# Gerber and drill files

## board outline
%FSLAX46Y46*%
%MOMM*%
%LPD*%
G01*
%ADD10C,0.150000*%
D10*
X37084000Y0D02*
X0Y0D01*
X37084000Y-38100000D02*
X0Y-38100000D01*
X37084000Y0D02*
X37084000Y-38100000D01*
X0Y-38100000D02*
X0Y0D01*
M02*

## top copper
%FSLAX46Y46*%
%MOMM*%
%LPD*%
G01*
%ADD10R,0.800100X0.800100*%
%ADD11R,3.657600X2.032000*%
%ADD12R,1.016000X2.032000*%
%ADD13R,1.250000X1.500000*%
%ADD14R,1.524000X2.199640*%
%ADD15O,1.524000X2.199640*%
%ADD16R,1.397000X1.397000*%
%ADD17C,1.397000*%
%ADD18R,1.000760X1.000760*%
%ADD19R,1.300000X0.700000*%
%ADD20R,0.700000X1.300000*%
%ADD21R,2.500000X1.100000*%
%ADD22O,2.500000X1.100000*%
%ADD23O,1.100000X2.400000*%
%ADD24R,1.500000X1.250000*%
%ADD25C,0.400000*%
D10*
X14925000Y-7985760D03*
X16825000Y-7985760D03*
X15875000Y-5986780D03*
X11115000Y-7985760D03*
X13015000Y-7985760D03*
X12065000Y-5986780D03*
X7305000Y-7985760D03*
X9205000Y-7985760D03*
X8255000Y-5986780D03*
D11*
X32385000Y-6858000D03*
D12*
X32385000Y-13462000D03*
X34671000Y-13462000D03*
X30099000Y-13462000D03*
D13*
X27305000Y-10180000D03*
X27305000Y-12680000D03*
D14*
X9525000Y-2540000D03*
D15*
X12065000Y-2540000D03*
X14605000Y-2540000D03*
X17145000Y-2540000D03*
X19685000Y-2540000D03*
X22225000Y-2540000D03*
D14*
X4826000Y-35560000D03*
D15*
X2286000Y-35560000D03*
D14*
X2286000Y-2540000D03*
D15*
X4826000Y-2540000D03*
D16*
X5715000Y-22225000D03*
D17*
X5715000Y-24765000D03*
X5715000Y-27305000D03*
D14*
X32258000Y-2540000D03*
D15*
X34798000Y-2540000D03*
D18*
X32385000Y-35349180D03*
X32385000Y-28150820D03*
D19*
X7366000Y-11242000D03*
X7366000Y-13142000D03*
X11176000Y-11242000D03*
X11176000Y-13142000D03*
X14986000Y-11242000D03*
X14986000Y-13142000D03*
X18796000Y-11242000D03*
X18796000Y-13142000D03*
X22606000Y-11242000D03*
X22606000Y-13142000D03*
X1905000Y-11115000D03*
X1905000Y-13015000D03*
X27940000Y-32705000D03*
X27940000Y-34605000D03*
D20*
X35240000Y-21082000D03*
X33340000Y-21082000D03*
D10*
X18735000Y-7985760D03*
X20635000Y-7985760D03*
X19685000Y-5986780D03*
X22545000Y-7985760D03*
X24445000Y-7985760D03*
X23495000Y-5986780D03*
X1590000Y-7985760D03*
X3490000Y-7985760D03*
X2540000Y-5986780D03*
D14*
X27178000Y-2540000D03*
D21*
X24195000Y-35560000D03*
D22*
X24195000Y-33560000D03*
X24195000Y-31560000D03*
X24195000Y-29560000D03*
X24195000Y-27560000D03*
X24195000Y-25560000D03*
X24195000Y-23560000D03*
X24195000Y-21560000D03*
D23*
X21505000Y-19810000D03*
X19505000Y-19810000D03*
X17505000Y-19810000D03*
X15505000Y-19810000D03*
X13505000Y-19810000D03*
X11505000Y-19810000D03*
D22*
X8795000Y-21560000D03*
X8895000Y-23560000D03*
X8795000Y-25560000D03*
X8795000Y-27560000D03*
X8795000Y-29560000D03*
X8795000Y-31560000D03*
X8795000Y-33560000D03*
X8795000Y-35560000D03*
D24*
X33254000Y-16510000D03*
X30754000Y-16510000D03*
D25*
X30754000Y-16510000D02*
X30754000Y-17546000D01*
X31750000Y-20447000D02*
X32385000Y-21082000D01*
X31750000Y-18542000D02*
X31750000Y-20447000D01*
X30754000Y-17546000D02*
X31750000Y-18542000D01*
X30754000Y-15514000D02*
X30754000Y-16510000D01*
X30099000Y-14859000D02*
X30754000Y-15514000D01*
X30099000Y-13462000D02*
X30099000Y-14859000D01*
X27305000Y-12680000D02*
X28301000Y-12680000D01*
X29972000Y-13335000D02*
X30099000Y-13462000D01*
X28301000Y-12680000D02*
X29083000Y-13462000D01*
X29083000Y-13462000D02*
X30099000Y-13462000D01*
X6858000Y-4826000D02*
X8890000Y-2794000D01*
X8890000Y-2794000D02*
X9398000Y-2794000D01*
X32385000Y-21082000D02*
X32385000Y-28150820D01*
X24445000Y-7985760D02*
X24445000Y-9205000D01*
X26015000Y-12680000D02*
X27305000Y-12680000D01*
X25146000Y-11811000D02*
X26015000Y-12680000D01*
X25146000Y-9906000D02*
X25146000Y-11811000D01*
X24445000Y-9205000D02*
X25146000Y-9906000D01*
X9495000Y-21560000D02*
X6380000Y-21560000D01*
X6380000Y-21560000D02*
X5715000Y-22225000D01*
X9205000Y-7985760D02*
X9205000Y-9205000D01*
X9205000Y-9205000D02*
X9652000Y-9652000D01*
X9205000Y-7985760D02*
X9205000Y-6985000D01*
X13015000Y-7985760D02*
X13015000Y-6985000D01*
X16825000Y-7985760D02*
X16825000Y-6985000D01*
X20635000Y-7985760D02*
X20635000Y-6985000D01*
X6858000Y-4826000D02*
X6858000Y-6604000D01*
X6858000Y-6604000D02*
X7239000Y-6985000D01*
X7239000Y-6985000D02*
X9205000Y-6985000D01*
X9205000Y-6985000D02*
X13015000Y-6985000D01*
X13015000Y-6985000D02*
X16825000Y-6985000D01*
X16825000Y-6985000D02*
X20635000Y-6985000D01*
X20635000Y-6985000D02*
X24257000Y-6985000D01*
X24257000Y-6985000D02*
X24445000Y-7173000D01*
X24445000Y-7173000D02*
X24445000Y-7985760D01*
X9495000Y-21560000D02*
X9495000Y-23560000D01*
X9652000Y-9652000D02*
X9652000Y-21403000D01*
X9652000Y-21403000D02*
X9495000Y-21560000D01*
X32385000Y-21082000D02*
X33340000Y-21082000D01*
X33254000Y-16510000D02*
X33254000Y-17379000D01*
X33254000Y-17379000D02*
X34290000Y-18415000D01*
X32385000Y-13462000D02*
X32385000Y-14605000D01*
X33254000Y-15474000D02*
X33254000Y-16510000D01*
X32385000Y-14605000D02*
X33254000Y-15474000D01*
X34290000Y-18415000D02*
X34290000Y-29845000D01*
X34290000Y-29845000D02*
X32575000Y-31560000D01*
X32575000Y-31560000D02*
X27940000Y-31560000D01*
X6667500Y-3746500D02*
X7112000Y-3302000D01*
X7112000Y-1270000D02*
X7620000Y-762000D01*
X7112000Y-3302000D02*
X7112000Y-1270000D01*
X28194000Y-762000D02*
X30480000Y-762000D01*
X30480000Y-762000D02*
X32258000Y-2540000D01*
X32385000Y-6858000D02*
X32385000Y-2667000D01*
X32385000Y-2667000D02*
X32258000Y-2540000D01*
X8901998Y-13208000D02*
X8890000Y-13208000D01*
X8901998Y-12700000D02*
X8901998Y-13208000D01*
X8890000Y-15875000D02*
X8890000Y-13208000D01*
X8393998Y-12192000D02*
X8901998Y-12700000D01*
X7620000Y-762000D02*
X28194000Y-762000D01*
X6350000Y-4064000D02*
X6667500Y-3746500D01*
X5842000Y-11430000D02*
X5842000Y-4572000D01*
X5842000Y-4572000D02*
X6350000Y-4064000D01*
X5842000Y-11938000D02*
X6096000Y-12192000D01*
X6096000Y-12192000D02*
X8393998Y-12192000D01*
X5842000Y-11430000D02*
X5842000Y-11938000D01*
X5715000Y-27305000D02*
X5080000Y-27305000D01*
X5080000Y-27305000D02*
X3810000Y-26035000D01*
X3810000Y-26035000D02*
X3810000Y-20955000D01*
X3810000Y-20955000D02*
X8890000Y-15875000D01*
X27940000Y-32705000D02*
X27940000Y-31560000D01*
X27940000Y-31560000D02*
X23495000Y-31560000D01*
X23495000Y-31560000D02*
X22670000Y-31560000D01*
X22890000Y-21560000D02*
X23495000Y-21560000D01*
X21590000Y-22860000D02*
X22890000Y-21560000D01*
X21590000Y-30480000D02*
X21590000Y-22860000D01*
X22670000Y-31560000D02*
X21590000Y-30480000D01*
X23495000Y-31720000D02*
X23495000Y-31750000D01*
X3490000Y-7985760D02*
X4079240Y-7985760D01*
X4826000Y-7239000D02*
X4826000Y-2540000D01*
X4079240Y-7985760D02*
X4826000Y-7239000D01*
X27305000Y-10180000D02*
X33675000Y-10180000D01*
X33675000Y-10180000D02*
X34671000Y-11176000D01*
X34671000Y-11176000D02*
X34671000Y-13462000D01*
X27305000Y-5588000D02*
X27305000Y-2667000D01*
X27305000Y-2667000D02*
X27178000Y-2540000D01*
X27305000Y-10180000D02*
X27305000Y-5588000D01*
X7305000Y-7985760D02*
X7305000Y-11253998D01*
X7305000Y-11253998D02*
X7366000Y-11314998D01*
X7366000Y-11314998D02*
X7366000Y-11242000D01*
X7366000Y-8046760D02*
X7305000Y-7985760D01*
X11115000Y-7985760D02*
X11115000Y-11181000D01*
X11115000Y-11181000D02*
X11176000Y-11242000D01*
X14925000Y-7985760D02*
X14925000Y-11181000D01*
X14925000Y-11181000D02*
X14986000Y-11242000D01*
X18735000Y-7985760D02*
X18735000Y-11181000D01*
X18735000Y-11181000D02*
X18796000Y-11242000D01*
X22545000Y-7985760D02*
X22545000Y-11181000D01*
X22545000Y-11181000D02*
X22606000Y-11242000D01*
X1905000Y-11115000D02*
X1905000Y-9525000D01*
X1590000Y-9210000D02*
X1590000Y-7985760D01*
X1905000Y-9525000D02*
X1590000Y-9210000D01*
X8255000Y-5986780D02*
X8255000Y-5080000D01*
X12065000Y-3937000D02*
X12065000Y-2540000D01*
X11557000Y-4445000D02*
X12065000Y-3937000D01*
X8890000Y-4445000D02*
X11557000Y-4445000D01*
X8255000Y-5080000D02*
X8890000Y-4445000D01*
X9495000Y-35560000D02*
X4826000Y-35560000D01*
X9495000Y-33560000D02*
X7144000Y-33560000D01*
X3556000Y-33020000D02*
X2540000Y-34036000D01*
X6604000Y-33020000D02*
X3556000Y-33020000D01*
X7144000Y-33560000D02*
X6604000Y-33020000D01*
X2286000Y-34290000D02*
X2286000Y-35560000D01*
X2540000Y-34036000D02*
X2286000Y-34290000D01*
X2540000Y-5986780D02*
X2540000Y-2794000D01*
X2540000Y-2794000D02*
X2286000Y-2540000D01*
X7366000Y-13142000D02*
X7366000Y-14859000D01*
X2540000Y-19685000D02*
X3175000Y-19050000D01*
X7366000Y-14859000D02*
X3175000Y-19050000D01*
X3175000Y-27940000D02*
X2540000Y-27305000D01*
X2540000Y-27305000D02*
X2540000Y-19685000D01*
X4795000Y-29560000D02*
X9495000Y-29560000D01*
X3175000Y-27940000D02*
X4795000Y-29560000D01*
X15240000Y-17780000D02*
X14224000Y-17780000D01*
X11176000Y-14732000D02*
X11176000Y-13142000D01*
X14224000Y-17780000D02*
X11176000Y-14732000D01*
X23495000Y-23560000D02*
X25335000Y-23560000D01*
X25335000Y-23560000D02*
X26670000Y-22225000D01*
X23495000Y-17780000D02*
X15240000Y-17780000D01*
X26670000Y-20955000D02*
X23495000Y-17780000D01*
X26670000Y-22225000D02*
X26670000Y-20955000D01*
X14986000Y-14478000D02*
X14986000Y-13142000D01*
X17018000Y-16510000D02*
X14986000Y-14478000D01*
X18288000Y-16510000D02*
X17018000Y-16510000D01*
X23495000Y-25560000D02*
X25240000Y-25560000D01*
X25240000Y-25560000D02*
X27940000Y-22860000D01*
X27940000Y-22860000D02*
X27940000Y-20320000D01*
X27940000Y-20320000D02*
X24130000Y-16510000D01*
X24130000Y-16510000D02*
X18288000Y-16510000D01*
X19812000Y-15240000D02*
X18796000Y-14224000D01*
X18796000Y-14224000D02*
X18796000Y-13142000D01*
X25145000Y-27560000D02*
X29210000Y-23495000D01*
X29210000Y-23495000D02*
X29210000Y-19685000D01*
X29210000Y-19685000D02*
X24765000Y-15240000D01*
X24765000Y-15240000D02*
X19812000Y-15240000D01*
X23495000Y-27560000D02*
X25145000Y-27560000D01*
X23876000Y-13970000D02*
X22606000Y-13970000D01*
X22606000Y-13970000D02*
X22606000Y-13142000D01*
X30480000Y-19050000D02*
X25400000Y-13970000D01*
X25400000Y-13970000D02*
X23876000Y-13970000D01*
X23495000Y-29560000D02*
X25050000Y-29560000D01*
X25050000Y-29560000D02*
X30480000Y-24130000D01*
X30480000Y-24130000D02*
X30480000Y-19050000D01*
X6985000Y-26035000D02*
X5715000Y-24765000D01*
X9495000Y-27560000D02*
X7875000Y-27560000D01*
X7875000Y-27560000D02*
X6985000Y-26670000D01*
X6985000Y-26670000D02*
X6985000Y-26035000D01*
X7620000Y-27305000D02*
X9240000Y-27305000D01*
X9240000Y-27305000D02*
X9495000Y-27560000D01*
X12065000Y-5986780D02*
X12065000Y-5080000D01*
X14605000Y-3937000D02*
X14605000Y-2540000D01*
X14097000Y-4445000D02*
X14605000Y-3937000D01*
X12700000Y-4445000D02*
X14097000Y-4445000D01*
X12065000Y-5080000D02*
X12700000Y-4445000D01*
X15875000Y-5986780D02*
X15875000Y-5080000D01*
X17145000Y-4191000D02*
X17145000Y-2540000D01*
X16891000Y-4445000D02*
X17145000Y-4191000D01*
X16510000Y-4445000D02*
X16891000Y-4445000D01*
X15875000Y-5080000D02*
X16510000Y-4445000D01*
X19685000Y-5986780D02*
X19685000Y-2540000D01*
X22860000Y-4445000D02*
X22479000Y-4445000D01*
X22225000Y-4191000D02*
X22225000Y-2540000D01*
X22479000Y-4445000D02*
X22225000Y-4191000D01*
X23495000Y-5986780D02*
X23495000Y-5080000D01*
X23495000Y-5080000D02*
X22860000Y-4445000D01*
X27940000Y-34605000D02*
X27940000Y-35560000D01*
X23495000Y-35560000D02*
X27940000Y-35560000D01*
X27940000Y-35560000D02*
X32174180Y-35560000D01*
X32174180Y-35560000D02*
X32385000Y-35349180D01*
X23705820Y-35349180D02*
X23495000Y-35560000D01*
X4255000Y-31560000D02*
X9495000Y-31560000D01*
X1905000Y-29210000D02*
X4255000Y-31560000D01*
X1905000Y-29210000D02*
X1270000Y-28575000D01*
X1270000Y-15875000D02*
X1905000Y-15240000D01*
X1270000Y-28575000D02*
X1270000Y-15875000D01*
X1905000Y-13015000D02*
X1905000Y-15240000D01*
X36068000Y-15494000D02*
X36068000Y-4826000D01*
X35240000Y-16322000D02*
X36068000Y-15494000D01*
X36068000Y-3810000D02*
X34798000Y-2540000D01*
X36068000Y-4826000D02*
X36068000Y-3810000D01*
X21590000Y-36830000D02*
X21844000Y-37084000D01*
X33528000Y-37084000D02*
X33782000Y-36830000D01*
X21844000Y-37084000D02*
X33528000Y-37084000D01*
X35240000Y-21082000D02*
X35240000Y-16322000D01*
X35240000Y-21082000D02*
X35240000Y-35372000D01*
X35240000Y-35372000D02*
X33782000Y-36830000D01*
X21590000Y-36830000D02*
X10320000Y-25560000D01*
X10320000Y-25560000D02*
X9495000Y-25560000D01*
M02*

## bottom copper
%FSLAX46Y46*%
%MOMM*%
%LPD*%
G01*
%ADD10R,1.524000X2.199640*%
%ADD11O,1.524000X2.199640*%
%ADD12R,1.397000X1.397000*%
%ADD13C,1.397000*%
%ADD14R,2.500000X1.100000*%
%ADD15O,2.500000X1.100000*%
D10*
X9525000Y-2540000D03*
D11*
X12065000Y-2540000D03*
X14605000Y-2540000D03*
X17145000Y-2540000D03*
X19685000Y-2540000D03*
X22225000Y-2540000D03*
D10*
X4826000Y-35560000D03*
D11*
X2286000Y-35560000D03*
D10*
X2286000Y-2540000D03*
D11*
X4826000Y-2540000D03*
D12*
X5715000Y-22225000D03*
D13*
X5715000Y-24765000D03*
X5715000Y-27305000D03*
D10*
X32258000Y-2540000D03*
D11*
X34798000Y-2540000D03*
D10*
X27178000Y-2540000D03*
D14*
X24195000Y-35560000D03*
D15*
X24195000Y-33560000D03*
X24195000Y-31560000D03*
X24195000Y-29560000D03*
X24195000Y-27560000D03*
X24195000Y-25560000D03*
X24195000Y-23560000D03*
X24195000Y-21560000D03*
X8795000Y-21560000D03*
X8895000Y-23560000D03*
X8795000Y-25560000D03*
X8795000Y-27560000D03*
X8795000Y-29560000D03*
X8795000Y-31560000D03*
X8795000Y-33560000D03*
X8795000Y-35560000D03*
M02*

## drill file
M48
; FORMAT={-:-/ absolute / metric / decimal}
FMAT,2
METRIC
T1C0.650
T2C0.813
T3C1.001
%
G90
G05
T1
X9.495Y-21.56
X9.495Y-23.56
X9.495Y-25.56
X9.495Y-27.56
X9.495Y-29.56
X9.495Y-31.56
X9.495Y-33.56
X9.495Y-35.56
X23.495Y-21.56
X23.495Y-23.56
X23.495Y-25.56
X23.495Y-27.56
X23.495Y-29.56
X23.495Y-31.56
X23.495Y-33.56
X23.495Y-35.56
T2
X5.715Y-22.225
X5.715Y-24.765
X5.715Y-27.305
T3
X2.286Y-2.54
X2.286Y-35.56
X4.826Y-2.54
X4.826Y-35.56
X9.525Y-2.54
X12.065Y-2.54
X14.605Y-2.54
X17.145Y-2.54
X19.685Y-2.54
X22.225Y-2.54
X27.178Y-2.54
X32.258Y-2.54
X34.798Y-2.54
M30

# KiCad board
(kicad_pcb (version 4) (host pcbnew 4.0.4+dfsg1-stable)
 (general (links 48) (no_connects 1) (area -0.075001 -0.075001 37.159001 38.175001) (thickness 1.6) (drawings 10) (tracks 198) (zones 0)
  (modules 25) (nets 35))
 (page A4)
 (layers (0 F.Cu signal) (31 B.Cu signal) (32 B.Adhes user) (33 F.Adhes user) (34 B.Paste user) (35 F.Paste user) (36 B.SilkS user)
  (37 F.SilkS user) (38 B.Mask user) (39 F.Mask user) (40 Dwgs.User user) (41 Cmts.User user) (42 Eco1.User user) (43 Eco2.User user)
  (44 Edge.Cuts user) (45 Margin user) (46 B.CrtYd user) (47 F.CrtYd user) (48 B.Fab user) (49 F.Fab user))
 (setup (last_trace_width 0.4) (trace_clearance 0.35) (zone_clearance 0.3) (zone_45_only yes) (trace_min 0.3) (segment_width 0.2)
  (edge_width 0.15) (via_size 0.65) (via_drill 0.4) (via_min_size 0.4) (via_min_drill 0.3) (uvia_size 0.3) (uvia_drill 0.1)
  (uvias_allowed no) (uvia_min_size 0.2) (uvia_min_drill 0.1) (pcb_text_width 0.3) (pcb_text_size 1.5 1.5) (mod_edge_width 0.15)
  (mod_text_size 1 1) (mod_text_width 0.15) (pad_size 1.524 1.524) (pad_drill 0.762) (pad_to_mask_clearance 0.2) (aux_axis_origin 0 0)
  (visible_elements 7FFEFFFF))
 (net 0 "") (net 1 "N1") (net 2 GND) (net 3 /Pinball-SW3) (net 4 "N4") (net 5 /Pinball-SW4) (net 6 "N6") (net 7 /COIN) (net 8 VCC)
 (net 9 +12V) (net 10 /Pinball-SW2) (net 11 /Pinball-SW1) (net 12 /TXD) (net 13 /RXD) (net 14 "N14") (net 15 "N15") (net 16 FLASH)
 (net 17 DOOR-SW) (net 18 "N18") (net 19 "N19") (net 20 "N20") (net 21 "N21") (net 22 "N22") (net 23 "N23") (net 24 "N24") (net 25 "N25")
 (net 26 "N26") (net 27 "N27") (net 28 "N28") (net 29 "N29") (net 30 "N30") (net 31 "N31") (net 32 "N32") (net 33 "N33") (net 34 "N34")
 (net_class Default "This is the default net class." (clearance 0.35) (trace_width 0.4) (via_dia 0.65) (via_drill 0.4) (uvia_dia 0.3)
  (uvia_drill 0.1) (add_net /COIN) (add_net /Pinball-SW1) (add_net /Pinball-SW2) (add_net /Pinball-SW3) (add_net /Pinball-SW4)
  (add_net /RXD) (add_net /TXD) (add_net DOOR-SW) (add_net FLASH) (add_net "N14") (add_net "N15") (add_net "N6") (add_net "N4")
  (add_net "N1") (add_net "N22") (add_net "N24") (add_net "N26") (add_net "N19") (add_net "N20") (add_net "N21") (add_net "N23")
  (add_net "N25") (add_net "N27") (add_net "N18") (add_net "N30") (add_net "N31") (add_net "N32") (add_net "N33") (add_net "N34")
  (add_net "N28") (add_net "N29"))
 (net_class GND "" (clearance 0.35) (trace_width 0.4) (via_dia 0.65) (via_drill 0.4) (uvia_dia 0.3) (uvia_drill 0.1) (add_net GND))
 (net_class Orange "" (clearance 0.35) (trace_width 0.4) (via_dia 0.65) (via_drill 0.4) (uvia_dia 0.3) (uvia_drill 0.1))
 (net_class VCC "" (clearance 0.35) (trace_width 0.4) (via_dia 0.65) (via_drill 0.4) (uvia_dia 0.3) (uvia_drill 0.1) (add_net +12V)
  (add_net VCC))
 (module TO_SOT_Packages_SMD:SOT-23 (layer F.Cu) (at 15.875 6.985)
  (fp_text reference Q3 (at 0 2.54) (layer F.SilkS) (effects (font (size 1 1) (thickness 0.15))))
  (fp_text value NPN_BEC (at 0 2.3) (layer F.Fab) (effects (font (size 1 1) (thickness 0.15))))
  (pad 1 smd rect (at -0.95 1.00076) (size 0.8001 0.8001) (layers F.Cu F.Paste F.Mask) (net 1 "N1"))
  (pad 2 smd rect (at 0.95 1.00076) (size 0.8001 0.8001) (layers F.Cu F.Paste F.Mask) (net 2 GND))
  (pad 3 smd rect (at 0 -0.99822) (size 0.8001 0.8001) (layers F.Cu F.Paste F.Mask) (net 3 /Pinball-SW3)))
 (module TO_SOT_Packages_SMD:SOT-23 (layer F.Cu) (at 12.065 6.985)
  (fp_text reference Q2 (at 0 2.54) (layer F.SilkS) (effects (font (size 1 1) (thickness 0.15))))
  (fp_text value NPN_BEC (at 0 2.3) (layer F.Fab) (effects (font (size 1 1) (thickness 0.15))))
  (pad 1 smd rect (at -0.95 1.00076) (size 0.8001 0.8001) (layers F.Cu F.Paste F.Mask) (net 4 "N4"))
  (pad 2 smd rect (at 0.95 1.00076) (size 0.8001 0.8001) (layers F.Cu F.Paste F.Mask) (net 2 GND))
  (pad 3 smd rect (at 0 -0.99822) (size 0.8001 0.8001) (layers F.Cu F.Paste F.Mask) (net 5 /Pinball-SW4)))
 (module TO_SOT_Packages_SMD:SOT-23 (layer F.Cu) (at 8.255 6.985)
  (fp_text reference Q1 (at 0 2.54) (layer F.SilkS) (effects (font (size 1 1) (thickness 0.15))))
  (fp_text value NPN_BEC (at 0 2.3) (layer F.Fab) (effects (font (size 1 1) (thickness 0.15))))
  (pad 1 smd rect (at -0.95 1.00076) (size 0.8001 0.8001) (layers F.Cu F.Paste F.Mask) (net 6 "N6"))
  (pad 2 smd rect (at 0.95 1.00076) (size 0.8001 0.8001) (layers F.Cu F.Paste F.Mask) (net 2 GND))
  (pad 3 smd rect (at 0 -0.99822) (size 0.8001 0.8001) (layers F.Cu F.Paste F.Mask) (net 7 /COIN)))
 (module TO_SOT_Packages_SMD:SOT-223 (layer F.Cu) (at 32.385 10.16)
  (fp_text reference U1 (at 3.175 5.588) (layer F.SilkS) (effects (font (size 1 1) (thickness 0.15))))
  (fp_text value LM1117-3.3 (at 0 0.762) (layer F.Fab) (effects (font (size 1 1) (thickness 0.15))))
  (pad 4 smd rect (at 0 -3.302) (size 3.6576 2.032) (layers F.Cu F.Paste F.Mask) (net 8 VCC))
  (pad 2 smd rect (at 0 3.302) (size 1.016 2.032) (layers F.Cu F.Paste F.Mask) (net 8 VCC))
  (pad 3 smd rect (at 2.286 3.302) (size 1.016 2.032) (layers F.Cu F.Paste F.Mask) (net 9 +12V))
  (pad 1 smd rect (at -2.286 3.302) (size 1.016 2.032) (layers F.Cu F.Paste F.Mask) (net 2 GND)))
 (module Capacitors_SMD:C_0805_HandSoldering (layer F.Cu) (at 27.305 11.43 270)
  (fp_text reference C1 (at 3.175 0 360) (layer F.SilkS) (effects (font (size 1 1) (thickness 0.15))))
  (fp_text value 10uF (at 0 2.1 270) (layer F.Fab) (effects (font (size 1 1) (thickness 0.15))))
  (pad 1 smd rect (at -1.25 0 270) (size 1.5 1.25) (layers F.Cu F.Paste F.Mask) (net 9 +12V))
  (pad 2 smd rect (at 1.25 0 270) (size 1.5 1.25) (layers F.Cu F.Paste F.Mask) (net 2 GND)))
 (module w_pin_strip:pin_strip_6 (layer F.Cu) (at 15.875 2.54)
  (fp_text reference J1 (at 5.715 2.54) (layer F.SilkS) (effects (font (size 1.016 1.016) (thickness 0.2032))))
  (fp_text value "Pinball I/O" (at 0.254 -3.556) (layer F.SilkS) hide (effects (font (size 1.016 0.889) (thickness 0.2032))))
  (pad 1 thru_hole rect (at -6.35 0) (size 1.524 2.19964) (drill 1.00076) (layers *.Cu *.Mask F.SilkS) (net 2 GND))
  (pad 2 thru_hole oval (at -3.81 0) (size 1.524 2.19964) (drill 1.00076) (layers *.Cu *.Mask F.SilkS) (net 7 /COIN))
  (pad 3 thru_hole oval (at -1.27 0) (size 1.524 2.19964) (drill 1.00076) (layers *.Cu *.Mask F.SilkS) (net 5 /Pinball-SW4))
  (pad 4 thru_hole oval (at 1.27 0) (size 1.524 2.19964) (drill 1.00076) (layers *.Cu *.Mask F.SilkS) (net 3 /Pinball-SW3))
  (pad 5 thru_hole oval (at 3.81 0) (size 1.524 2.19964) (drill 1.00076) (layers *.Cu *.Mask F.SilkS) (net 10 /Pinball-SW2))
  (pad 6 thru_hole oval (at 6.35 0) (size 1.524 2.19964) (drill 1.00076) (layers *.Cu *.Mask F.SilkS) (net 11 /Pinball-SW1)))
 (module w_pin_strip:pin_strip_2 (layer F.Cu) (at 3.556 35.56 180)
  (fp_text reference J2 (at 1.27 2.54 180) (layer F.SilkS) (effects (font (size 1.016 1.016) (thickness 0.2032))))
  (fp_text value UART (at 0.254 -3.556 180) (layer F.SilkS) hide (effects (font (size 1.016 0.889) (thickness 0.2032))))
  (pad 1 thru_hole rect (at -1.27 0 180) (size 1.524 2.19964) (drill 1.00076) (layers *.Cu *.Mask F.SilkS) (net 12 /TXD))
  (pad 2 thru_hole oval (at 1.27 0 180) (size 1.524 2.19964) (drill 1.00076) (layers *.Cu *.Mask F.SilkS) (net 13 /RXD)))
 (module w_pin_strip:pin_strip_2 (layer F.Cu) (at 3.556 2.54)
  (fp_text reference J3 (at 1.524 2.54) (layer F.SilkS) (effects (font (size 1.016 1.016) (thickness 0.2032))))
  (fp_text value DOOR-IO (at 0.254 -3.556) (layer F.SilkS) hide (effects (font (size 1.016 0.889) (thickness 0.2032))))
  (pad 1 thru_hole rect (at -1.27 0) (size 1.524 2.19964) (drill 1.00076) (layers *.Cu *.Mask F.SilkS) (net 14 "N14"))
  (pad 2 thru_hole oval (at 1.27 0) (size 1.524 2.19964) (drill 1.00076) (layers *.Cu *.Mask F.SilkS) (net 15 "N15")))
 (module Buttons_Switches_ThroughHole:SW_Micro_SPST (layer F.Cu) (at 5.715 24.765 270)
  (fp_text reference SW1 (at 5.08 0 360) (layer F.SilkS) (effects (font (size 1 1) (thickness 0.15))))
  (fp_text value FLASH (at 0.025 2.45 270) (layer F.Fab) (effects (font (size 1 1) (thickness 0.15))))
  (pad 1 thru_hole rect (at -2.54 0 270) (size 1.397 1.397) (drill 0.8128) (layers *.Cu *.Mask F.SilkS) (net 2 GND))
  (pad 2 thru_hole circle (at 0 0 270) (size 1.397 1.397) (drill 0.8128) (layers *.Cu *.Mask F.SilkS) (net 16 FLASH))
  (pad 3 thru_hole circle (at 2.54 0 270) (size 1.397 1.397) (drill 0.8128) (layers *.Cu *.Mask F.SilkS) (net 8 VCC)))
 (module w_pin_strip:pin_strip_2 (layer F.Cu) (at 33.528 2.54)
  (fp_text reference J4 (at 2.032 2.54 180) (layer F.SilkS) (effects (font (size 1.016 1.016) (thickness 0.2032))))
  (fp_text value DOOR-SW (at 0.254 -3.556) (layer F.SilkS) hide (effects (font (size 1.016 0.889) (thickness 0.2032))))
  (pad 1 thru_hole rect (at -1.27 0) (size 1.524 2.19964) (drill 1.00076) (layers *.Cu *.Mask F.SilkS) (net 8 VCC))
  (pad 2 thru_hole oval (at 1.27 0) (size 1.524 2.19964) (drill 1.00076) (layers *.Cu *.Mask F.SilkS) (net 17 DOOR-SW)))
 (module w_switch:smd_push (layer F.Cu) (at 32.385 31.75 90) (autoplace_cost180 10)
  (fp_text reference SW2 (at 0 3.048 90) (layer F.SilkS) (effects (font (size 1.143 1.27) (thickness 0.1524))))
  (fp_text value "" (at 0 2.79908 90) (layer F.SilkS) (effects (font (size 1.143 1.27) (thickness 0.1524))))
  (pad 1 smd rect (at -3.59918 0 90) (size 1.00076 1.00076) (layers F.Cu F.Paste F.Mask) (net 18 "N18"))
  (pad 2 smd rect (at 3.59918 0 90) (size 1.00076 1.00076) (layers F.Cu F.Paste F.Mask) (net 2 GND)))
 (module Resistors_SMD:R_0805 (layer F.Cu) (at 7.366 12.192 270)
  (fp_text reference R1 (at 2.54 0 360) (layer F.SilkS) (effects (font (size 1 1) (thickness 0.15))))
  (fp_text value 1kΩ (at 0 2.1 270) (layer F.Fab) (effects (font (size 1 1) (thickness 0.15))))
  (pad 1 smd rect (at -0.95 0 270) (size 0.7 1.3) (layers F.Cu F.Paste F.Mask) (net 6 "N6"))
  (pad 2 smd rect (at 0.95 0 270) (size 0.7 1.3) (layers F.Cu F.Paste F.Mask) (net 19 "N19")))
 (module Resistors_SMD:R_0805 (layer F.Cu) (at 11.176 12.192 270)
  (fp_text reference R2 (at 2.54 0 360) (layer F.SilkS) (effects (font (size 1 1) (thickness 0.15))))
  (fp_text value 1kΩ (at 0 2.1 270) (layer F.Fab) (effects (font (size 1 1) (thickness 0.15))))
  (pad 1 smd rect (at -0.95 0 270) (size 0.7 1.3) (layers F.Cu F.Paste F.Mask) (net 4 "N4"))
  (pad 2 smd rect (at 0.95 0 270) (size 0.7 1.3) (layers F.Cu F.Paste F.Mask) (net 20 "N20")))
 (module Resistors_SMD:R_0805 (layer F.Cu) (at 14.986 12.192 270)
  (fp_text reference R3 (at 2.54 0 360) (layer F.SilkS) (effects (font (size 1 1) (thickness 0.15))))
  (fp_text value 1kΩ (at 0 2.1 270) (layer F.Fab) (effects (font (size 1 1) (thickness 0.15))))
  (pad 1 smd rect (at -0.95 0 270) (size 0.7 1.3) (layers F.Cu F.Paste F.Mask) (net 1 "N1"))
  (pad 2 smd rect (at 0.95 0 270) (size 0.7 1.3) (layers F.Cu F.Paste F.Mask) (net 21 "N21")))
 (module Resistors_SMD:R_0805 (layer F.Cu) (at 18.796 12.192 270)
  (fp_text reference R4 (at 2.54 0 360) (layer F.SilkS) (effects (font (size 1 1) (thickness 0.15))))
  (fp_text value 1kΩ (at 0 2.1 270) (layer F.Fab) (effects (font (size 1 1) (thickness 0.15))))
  (pad 1 smd rect (at -0.95 0 270) (size 0.7 1.3) (layers F.Cu F.Paste F.Mask) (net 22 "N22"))
  (pad 2 smd rect (at 0.95 0 270) (size 0.7 1.3) (layers F.Cu F.Paste F.Mask) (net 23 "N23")))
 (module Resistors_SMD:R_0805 (layer F.Cu) (at 22.606 12.192 270)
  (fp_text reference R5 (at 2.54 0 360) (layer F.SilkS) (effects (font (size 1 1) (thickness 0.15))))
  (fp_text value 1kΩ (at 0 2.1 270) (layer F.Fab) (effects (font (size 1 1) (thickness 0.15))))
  (pad 1 smd rect (at -0.95 0 270) (size 0.7 1.3) (layers F.Cu F.Paste F.Mask) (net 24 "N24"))
  (pad 2 smd rect (at 0.95 0 270) (size 0.7 1.3) (layers F.Cu F.Paste F.Mask) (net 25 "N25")))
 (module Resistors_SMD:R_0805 (layer F.Cu) (at 1.905 12.065 270)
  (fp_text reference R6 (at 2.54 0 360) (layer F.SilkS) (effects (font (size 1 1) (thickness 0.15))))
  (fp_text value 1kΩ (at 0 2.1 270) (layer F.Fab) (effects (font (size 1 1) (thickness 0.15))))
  (pad 1 smd rect (at -0.95 0 270) (size 0.7 1.3) (layers F.Cu F.Paste F.Mask) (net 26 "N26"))
  (pad 2 smd rect (at 0.95 0 270) (size 0.7 1.3) (layers F.Cu F.Paste F.Mask) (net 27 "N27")))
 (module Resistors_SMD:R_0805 (layer F.Cu) (at 27.94 33.655 270)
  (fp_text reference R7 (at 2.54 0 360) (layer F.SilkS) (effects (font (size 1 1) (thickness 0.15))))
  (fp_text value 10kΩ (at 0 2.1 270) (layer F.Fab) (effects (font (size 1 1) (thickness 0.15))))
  (pad 1 smd rect (at -0.95 0 270) (size 0.7 1.3) (layers F.Cu F.Paste F.Mask) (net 8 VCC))
  (pad 2 smd rect (at 0.95 0 270) (size 0.7 1.3) (layers F.Cu F.Paste F.Mask) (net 18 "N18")))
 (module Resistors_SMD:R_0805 (layer F.Cu) (at 34.29 21.082 180)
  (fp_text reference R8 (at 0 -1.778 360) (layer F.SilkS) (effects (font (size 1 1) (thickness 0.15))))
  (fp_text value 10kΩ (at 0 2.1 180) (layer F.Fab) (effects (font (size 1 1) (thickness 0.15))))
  (pad 1 smd rect (at -0.95 0 180) (size 0.7 1.3) (layers F.Cu F.Paste F.Mask) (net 17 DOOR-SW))
  (pad 2 smd rect (at 0.95 0 180) (size 0.7 1.3) (layers F.Cu F.Paste F.Mask) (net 2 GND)))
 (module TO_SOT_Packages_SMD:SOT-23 (layer F.Cu) (at 19.685 6.985)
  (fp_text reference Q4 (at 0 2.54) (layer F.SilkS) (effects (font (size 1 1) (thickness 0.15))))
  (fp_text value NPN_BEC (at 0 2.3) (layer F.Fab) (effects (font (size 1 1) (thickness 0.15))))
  (pad 1 smd rect (at -0.95 1.00076) (size 0.8001 0.8001) (layers F.Cu F.Paste F.Mask) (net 22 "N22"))
  (pad 2 smd rect (at 0.95 1.00076) (size 0.8001 0.8001) (layers F.Cu F.Paste F.Mask) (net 2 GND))
  (pad 3 smd rect (at 0 -0.99822) (size 0.8001 0.8001) (layers F.Cu F.Paste F.Mask) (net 10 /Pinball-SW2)))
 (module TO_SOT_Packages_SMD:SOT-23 (layer F.Cu) (at 23.495 6.985)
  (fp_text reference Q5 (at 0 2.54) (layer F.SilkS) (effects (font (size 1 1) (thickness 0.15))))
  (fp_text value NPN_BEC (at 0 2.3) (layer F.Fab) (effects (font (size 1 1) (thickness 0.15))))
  (pad 1 smd rect (at -0.95 1.00076) (size 0.8001 0.8001) (layers F.Cu F.Paste F.Mask) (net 24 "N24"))
  (pad 2 smd rect (at 0.95 1.00076) (size 0.8001 0.8001) (layers F.Cu F.Paste F.Mask) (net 2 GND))
  (pad 3 smd rect (at 0 -0.99822) (size 0.8001 0.8001) (layers F.Cu F.Paste F.Mask) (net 11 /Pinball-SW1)))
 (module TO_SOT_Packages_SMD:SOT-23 (layer F.Cu) (at 2.54 6.985)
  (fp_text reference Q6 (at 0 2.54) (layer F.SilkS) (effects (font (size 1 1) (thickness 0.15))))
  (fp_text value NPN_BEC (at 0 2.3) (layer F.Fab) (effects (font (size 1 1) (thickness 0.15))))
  (pad 1 smd rect (at -0.95 1.00076) (size 0.8001 0.8001) (layers F.Cu F.Paste F.Mask) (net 26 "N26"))
  (pad 2 smd rect (at 0.95 1.00076) (size 0.8001 0.8001) (layers F.Cu F.Paste F.Mask) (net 15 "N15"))
  (pad 3 smd rect (at 0 -0.99822) (size 0.8001 0.8001) (layers F.Cu F.Paste F.Mask) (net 14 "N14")))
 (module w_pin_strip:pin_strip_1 (layer F.Cu) (at 27.178 2.54)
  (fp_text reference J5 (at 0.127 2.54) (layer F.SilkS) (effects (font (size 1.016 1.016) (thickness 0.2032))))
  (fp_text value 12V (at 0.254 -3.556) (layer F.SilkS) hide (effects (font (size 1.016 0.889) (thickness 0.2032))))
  (pad 1 thru_hole rect (at 0 0) (size 1.524 2.19964) (drill 1.00076) (layers *.Cu *.Mask F.SilkS) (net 9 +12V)))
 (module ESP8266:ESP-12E (layer F.Cu) (at 23.495 35.56 180)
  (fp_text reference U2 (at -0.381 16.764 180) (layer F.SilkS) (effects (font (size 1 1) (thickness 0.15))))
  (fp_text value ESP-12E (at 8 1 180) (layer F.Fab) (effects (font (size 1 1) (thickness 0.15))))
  (pad 1 thru_hole rect (at 0 0 180) (size 2.5 1.1) (drill 0.65 (offset -0.7 0)) (layers *.Cu *.Mask F.SilkS) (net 18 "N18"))
  (pad 2 thru_hole oval (at 0 2 180) (size 2.5 1.1) (drill 0.65 (offset -0.7 0)) (layers *.Cu *.Mask F.SilkS) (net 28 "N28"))
  (pad 3 thru_hole oval (at 0 4 180) (size 2.5 1.1) (drill 0.65 (offset -0.7 0)) (layers *.Cu *.Mask F.SilkS) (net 8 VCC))
  (pad 4 thru_hole oval (at 0 6 180) (size 2.5 1.1) (drill 0.65 (offset -0.7 0)) (layers *.Cu *.Mask F.SilkS) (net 25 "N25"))
  (pad 5 thru_hole oval (at 0 8 180) (size 2.5 1.1) (drill 0.65 (offset -0.7 0)) (layers *.Cu *.Mask F.SilkS) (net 23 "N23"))
  (pad 6 thru_hole oval (at 0 10 180) (size 2.5 1.1) (drill 0.65 (offset -0.7 0)) (layers *.Cu *.Mask F.SilkS) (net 21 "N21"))
  (pad 7 thru_hole oval (at 0 12 180) (size 2.5 1.1) (drill 0.65 (offset -0.7 0)) (layers *.Cu *.Mask F.SilkS) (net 20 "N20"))
  (pad 8 thru_hole oval (at 0 14 180) (size 2.5 1.1) (drill 0.65 (offset -0.7 0)) (layers *.Cu *.Mask F.SilkS) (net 8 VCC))
  (pad 9 smd oval (at 1.99 15.75 270) (size 2.4 1.1) (layers F.Cu F.Paste F.Mask) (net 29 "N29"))
  (pad 10 smd oval (at 3.99 15.75 270) (size 2.4 1.1) (layers F.Cu F.Paste F.Mask) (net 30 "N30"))
  (pad 11 smd oval (at 5.99 15.75 270) (size 2.4 1.1) (layers F.Cu F.Paste F.Mask) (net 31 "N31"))
  (pad 12 smd oval (at 7.99 15.75 270) (size 2.4 1.1) (layers F.Cu F.Paste F.Mask) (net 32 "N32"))
  (pad 13 smd oval (at 9.99 15.75 270) (size 2.4 1.1) (layers F.Cu F.Paste F.Mask) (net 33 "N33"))
  (pad 14 smd oval (at 11.99 15.75 270) (size 2.4 1.1) (layers F.Cu F.Paste F.Mask) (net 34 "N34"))
  (pad 15 thru_hole oval (at 14 14 180) (size 2.5 1.1) (drill 0.65 (offset 0.7 0)) (layers *.Cu *.Mask F.SilkS) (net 2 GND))
  (pad 16 thru_hole oval (at 14 12 180) (size 2.5 1.1) (drill 0.65 (offset 0.6 0)) (layers *.Cu *.Mask F.SilkS) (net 2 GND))
  (pad 17 thru_hole oval (at 14 10 180) (size 2.5 1.1) (drill 0.65 (offset 0.7 0)) (layers *.Cu *.Mask F.SilkS) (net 17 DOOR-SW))
  (pad 18 thru_hole oval (at 14 8 180) (size 2.5 1.1) (drill 0.65 (offset 0.7 0)) (layers *.Cu *.Mask F.SilkS) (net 16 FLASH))
  (pad 19 thru_hole oval (at 14 6 180) (size 2.5 1.1) (drill 0.65 (offset 0.7 0)) (layers *.Cu *.Mask F.SilkS) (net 19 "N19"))
  (pad 20 thru_hole oval (at 14 4 180) (size 2.5 1.1) (drill 0.65 (offset 0.7 0)) (layers *.Cu *.Mask F.SilkS) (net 27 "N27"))
  (pad 21 thru_hole oval (at 14 2 180) (size 2.5 1.1) (drill 0.65 (offset 0.7 0)) (layers *.Cu *.Mask F.SilkS) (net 13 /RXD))
  (pad 22 thru_hole oval (at 14 0 180) (size 2.5 1.1) (drill 0.65 (offset 0.7 0)) (layers *.Cu *.Mask F.SilkS) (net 12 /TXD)))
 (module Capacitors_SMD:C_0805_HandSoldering (layer F.Cu) (at 32.004 16.51 180)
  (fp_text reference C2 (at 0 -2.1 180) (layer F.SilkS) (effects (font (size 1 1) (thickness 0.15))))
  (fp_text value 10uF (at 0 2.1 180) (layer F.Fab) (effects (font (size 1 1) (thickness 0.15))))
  (pad 1 smd rect (at -1.25 0 180) (size 1.5 1.25) (layers F.Cu F.Paste F.Mask) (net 8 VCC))
  (pad 2 smd rect (at 1.25 0 180) (size 1.5 1.25) (layers F.Cu F.Paste F.Mask) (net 2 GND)))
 (gr_line (start 37.084 0) (end 0 0) (angle 90) (layer Edge.Cuts) (width 0.15))
 (gr_line (start 37.084 38.1) (end 0 38.1) (angle 90) (layer Edge.Cuts) (width 0.15))
 (gr_line (start 37.084 0) (end 37.084 38.1) (angle 90) (layer Edge.Cuts) (width 0.15))
 (gr_line (start 0 38.1) (end 0 0) (angle 90) (layer Edge.Cuts) (width 0.15))
 (segment (start 30.754 16.51) (end 30.754 17.546) (width 0.4) (layer F.Cu) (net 2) (status 400000))
 (segment (start 31.75 20.447) (end 32.385 21.082) (width 0.4) (layer F.Cu) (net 2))
 (segment (start 31.75 18.542) (end 31.75 20.447) (width 0.4) (layer F.Cu) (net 2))
 (segment (start 30.754 17.546) (end 31.75 18.542) (width 0.4) (layer F.Cu) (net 2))
 (segment (start 30.754 15.514) (end 30.754 16.51) (width 0.4) (layer F.Cu) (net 2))
 (segment (start 30.099 14.859) (end 30.754 15.514) (width 0.4) (layer F.Cu) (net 2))
 (segment (start 30.099 13.462) (end 30.099 14.859) (width 0.4) (layer F.Cu) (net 2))
 (segment (start 27.305 12.68) (end 28.301 12.68) (width 0.4) (layer F.Cu) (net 2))
 (segment (start 29.972 13.335) (end 30.099 13.462) (width 0.4) (layer F.Cu) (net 2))
 (segment (start 28.301 12.68) (end 29.083 13.462) (width 0.4) (layer F.Cu) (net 2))
 (segment (start 29.083 13.462) (end 30.099 13.462) (width 0.4) (layer F.Cu) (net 2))
 (segment (start 6.858 4.826) (end 8.89 2.794) (width 0.4) (layer F.Cu) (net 2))
 (segment (start 8.89 2.794) (end 9.398 2.794) (width 0.4) (layer F.Cu) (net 2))
 (segment (start 32.385 21.082) (end 32.385 28.15082) (width 0.4) (layer F.Cu) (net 2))
 (segment (start 24.445 7.98576) (end 24.445 9.205) (width 0.4) (layer F.Cu) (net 2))
 (segment (start 26.015 12.68) (end 27.305 12.68) (width 0.4) (layer F.Cu) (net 2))
 (segment (start 25.146 11.811) (end 26.015 12.68) (width 0.4) (layer F.Cu) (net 2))
 (segment (start 25.146 9.906) (end 25.146 11.811) (width 0.4) (layer F.Cu) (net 2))
 (segment (start 24.445 9.205) (end 25.146 9.906) (width 0.4) (layer F.Cu) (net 2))
 (segment (start 9.495 21.56) (end 6.38 21.56) (width 0.4) (layer F.Cu) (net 2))
 (segment (start 6.38 21.56) (end 5.715 22.225) (width 0.4) (layer F.Cu) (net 2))
 (segment (start 9.205 7.98576) (end 9.205 9.205) (width 0.4) (layer F.Cu) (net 2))
 (segment (start 9.205 9.205) (end 9.652 9.652) (width 0.4) (layer F.Cu) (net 2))
 (segment (start 9.205 7.98576) (end 9.205 6.985) (width 0.4) (layer F.Cu) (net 2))
 (segment (start 13.015 7.98576) (end 13.015 6.985) (width 0.4) (layer F.Cu) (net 2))
 (segment (start 16.825 7.98576) (end 16.825 6.985) (width 0.4) (layer F.Cu) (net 2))
 (segment (start 20.635 7.98576) (end 20.635 6.985) (width 0.4) (layer F.Cu) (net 2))
 (segment (start 6.858 4.826) (end 6.858 6.604) (width 0.4) (layer F.Cu) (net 2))
 (segment (start 6.858 6.604) (end 7.239 6.985) (width 0.4) (layer F.Cu) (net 2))
 (segment (start 7.239 6.985) (end 9.205 6.985) (width 0.4) (layer F.Cu) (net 2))
 (segment (start 9.205 6.985) (end 13.015 6.985) (width 0.4) (layer F.Cu) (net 2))
 (segment (start 13.015 6.985) (end 16.825 6.985) (width 0.4) (layer F.Cu) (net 2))
 (segment (start 16.825 6.985) (end 20.635 6.985) (width 0.4) (layer F.Cu) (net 2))
 (segment (start 20.635 6.985) (end 24.257 6.985) (width 0.4) (layer F.Cu) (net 2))
 (segment (start 24.257 6.985) (end 24.445 7.173) (width 0.4) (layer F.Cu) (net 2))
 (segment (start 24.445 7.173) (end 24.445 7.98576) (width 0.4) (layer F.Cu) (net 2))
 (segment (start 9.495 21.56) (end 9.495 23.56) (width 0.4) (layer F.Cu) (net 2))
 (segment (start 9.652 9.652) (end 9.652 21.403) (width 0.4) (layer F.Cu) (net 2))
 (segment (start 9.652 21.403) (end 9.495 21.56) (width 0.4) (layer F.Cu) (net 2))
 (segment (start 32.385 21.082) (end 33.34 21.082) (width 0.4) (layer F.Cu) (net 2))
 (segment (start 33.254 16.51) (end 33.254 17.379) (width 0.4) (layer F.Cu) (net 8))
 (segment (start 33.254 17.379) (end 34.29 18.415) (width 0.4) (layer F.Cu) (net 8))
 (segment (start 32.385 13.462) (end 32.385 14.605) (width 0.4) (layer F.Cu) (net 8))
 (segment (start 33.254 15.474) (end 33.254 16.51) (width 0.4) (layer F.Cu) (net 8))
 (segment (start 32.385 14.605) (end 33.254 15.474) (width 0.4) (layer F.Cu) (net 8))
 (segment (start 34.29 18.415) (end 34.29 29.845) (width 0.4) (layer F.Cu) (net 8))
 (segment (start 34.29 29.845) (end 32.575 31.56) (width 0.4) (layer F.Cu) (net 8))
 (segment (start 32.575 31.56) (end 27.94 31.56) (width 0.4) (layer F.Cu) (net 8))
 (segment (start 6.6675 3.7465) (end 7.112 3.302) (width 0.4) (layer F.Cu) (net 8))
 (segment (start 7.112 1.27) (end 7.62 0.762) (width 0.4) (layer F.Cu) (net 8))
 (segment (start 7.112 3.302) (end 7.112 1.27) (width 0.4) (layer F.Cu) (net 8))
 (segment (start 28.194 0.762) (end 30.48 0.762) (width 0.4) (layer F.Cu) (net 8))
 (segment (start 30.48 0.762) (end 32.258 2.54) (width 0.4) (layer F.Cu) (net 8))
 (segment (start 32.385 6.858) (end 32.385 2.667) (width 0.4) (layer F.Cu) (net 8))
 (segment (start 32.385 2.667) (end 32.258 2.54) (width 0.4) (layer F.Cu) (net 8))
 (segment (start 8.901998 13.208) (end 8.89 13.208) (width 0.4) (layer F.Cu) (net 8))
 (segment (start 8.901998 12.7) (end 8.901998 13.208) (width 0.4) (layer F.Cu) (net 8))
 (segment (start 8.89 15.875) (end 8.89 13.208) (width 0.4) (layer F.Cu) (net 8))
 (segment (start 8.393998 12.192) (end 8.901998 12.7) (width 0.4) (layer F.Cu) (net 8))
 (segment (start 7.62 0.762) (end 28.194 0.762) (width 0.4) (layer F.Cu) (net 8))
 (segment (start 6.35 4.064) (end 6.6675 3.7465) (width 0.4) (layer F.Cu) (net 8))
 (segment (start 5.842 11.43) (end 5.842 4.572) (width 0.4) (layer F.Cu) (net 8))
 (segment (start 5.842 4.572) (end 6.35 4.064) (width 0.4) (layer F.Cu) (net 8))
 (segment (start 5.842 11.938) (end 6.096 12.192) (width 0.4) (layer F.Cu) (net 8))
 (segment (start 6.096 12.192) (end 8.393998 12.192) (width 0.4) (layer F.Cu) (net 8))
 (segment (start 5.842 11.43) (end 5.842 11.938) (width 0.4) (layer F.Cu) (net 8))
 (segment (start 5.715 27.305) (end 5.08 27.305) (width 0.4) (layer F.Cu) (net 8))
 (segment (start 5.08 27.305) (end 3.81 26.035) (width 0.4) (layer F.Cu) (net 8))
 (segment (start 3.81 26.035) (end 3.81 20.955) (width 0.4) (layer F.Cu) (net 8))
 (segment (start 3.81 20.955) (end 8.89 15.875) (width 0.4) (layer F.Cu) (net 8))
 (segment (start 27.94 32.705) (end 27.94 31.56) (width 0.4) (layer F.Cu) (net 8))
 (segment (start 27.94 31.56) (end 23.495 31.56) (width 0.4) (layer F.Cu) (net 8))
 (segment (start 23.495 31.56) (end 22.67 31.56) (width 0.4) (layer F.Cu) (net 8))
 (segment (start 22.89 21.56) (end 23.495 21.56) (width 0.4) (layer F.Cu) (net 8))
 (segment (start 21.59 22.86) (end 22.89 21.56) (width 0.4) (layer F.Cu) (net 8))
 (segment (start 21.59 30.48) (end 21.59 22.86) (width 0.4) (layer F.Cu) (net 8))
 (segment (start 22.67 31.56) (end 21.59 30.48) (width 0.4) (layer F.Cu) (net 8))
 (segment (start 23.495 31.72) (end 23.495 31.75) (width 0.4) (layer F.Cu) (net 8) (status 30))
 (segment (start 3.49 7.98576) (end 4.07924 7.98576) (width 0.4) (layer F.Cu) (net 15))
 (segment (start 4.826 7.239) (end 4.826 2.54) (width 0.4) (layer F.Cu) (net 15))
 (segment (start 4.07924 7.98576) (end 4.826 7.239) (width 0.4) (layer F.Cu) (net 15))
 (segment (start 27.305 10.18) (end 33.675 10.18) (width 0.4) (layer F.Cu) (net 9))
 (segment (start 33.675 10.18) (end 34.671 11.176) (width 0.4) (layer F.Cu) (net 9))
 (segment (start 34.671 11.176) (end 34.671 13.462) (width 0.4) (layer F.Cu) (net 9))
 (segment (start 27.305 5.588) (end 27.305 2.667) (width 0.4) (layer F.Cu) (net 9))
 (segment (start 27.305 2.667) (end 27.178 2.54) (width 0.4) (layer F.Cu) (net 9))
 (segment (start 27.305 10.18) (end 27.305 5.588) (width 0.4) (layer F.Cu) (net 9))
 (segment (start 7.305 7.98576) (end 7.305 11.253998) (width 0.4) (layer F.Cu) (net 6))
 (segment (start 7.305 11.253998) (end 7.366 11.314998) (width 0.4) (layer F.Cu) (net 6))
 (segment (start 7.366 11.314998) (end 7.366 11.242) (width 0.4) (layer F.Cu) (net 6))
 (segment (start 7.366 8.04676) (end 7.305 7.98576) (width 0.4) (layer F.Cu) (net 6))
 (segment (start 11.115 7.98576) (end 11.115 11.181) (width 0.4) (layer F.Cu) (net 4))
 (segment (start 11.115 11.181) (end 11.176 11.242) (width 0.4) (layer F.Cu) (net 4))
 (segment (start 14.925 7.98576) (end 14.925 11.181) (width 0.4) (layer F.Cu) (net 1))
 (segment (start 14.925 11.181) (end 14.986 11.242) (width 0.4) (layer F.Cu) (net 1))
 (segment (start 18.735 7.98576) (end 18.735 11.181) (width 0.4) (layer F.Cu) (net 22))
 (segment (start 18.735 11.181) (end 18.796 11.242) (width 0.4) (layer F.Cu) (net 22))
 (segment (start 22.545 7.98576) (end 22.545 11.181) (width 0.4) (layer F.Cu) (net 24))
 (segment (start 22.545 11.181) (end 22.606 11.242) (width 0.4) (layer F.Cu) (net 24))
 (segment (start 1.905 11.115) (end 1.905 9.525) (width 0.4) (layer F.Cu) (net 26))
 (segment (start 1.59 9.21) (end 1.59 7.98576) (width 0.4) (layer F.Cu) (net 26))
 (segment (start 1.905 9.525) (end 1.59 9.21) (width 0.4) (layer F.Cu) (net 26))
 (segment (start 8.255 5.98678) (end 8.255 5.08) (width 0.4) (layer F.Cu) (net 7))
 (segment (start 12.065 3.937) (end 12.065 2.54) (width 0.4) (layer F.Cu) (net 7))
 (segment (start 11.557 4.445) (end 12.065 3.937) (width 0.4) (layer F.Cu) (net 7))
 (segment (start 8.89 4.445) (end 11.557 4.445) (width 0.4) (layer F.Cu) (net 7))
 (segment (start 8.255 5.08) (end 8.89 4.445) (width 0.4) (layer F.Cu) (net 7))
 (segment (start 9.495 35.56) (end 4.826 35.56) (width 0.4) (layer F.Cu) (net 12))
 (segment (start 9.495 33.56) (end 7.144 33.56) (width 0.4) (layer F.Cu) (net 13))
 (segment (start 3.556 33.02) (end 2.54 34.036) (width 0.4) (layer F.Cu) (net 13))
 (segment (start 6.604 33.02) (end 3.556 33.02) (width 0.4) (layer F.Cu) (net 13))
 (segment (start 7.144 33.56) (end 6.604 33.02) (width 0.4) (layer F.Cu) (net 13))
 (segment (start 2.286 34.29) (end 2.286 35.56) (width 0.4) (layer F.Cu) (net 13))
 (segment (start 2.54 34.036) (end 2.286 34.29) (width 0.4) (layer F.Cu) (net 13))
 (segment (start 2.54 5.98678) (end 2.54 2.794) (width 0.4) (layer F.Cu) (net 14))
 (segment (start 2.54 2.794) (end 2.286 2.54) (width 0.4) (layer F.Cu) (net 14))
 (segment (start 7.366 13.142) (end 7.366 14.859) (width 0.4) (layer F.Cu) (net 19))
 (segment (start 2.54 19.685) (end 3.175 19.05) (width 0.4) (layer F.Cu) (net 19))
 (segment (start 7.366 14.859) (end 3.175 19.05) (width 0.4) (layer F.Cu) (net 19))
 (segment (start 3.175 27.94) (end 2.54 27.305) (width 0.4) (layer F.Cu) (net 19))
 (segment (start 2.54 27.305) (end 2.54 19.685) (width 0.4) (layer F.Cu) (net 19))
 (segment (start 4.795 29.56) (end 9.495 29.56) (width 0.4) (layer F.Cu) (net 19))
 (segment (start 3.175 27.94) (end 4.795 29.56) (width 0.4) (layer F.Cu) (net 19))
 (segment (start 15.24 17.78) (end 14.224 17.78) (width 0.4) (layer F.Cu) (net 20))
 (segment (start 11.176 14.732) (end 11.176 13.142) (width 0.4) (layer F.Cu) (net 20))
 (segment (start 14.224 17.78) (end 11.176 14.732) (width 0.4) (layer F.Cu) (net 20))
 (segment (start 23.495 23.56) (end 25.335 23.56) (width 0.4) (layer F.Cu) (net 20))
 (segment (start 25.335 23.56) (end 26.67 22.225) (width 0.4) (layer F.Cu) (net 20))
 (segment (start 23.495 17.78) (end 15.24 17.78) (width 0.4) (layer F.Cu) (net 20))
 (segment (start 26.67 20.955) (end 23.495 17.78) (width 0.4) (layer F.Cu) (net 20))
 (segment (start 26.67 22.225) (end 26.67 20.955) (width 0.4) (layer F.Cu) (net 20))
 (segment (start 14.986 14.478) (end 14.986 13.142) (width 0.4) (layer F.Cu) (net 21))
 (segment (start 17.018 16.51) (end 14.986 14.478) (width 0.4) (layer F.Cu) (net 21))
 (segment (start 18.288 16.51) (end 17.018 16.51) (width 0.4) (layer F.Cu) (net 21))
 (segment (start 23.495 25.56) (end 25.24 25.56) (width 0.4) (layer F.Cu) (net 21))
 (segment (start 25.24 25.56) (end 27.94 22.86) (width 0.4) (layer F.Cu) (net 21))
 (segment (start 27.94 22.86) (end 27.94 20.32) (width 0.4) (layer F.Cu) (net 21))
 (segment (start 27.94 20.32) (end 24.13 16.51) (width 0.4) (layer F.Cu) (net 21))
 (segment (start 24.13 16.51) (end 18.288 16.51) (width 0.4) (layer F.Cu) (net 21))
 (segment (start 19.812 15.24) (end 18.796 14.224) (width 0.4) (layer F.Cu) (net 23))
 (segment (start 18.796 14.224) (end 18.796 13.142) (width 0.4) (layer F.Cu) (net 23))
 (segment (start 25.145 27.56) (end 29.21 23.495) (width 0.4) (layer F.Cu) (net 23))
 (segment (start 29.21 23.495) (end 29.21 19.685) (width 0.4) (layer F.Cu) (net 23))
 (segment (start 29.21 19.685) (end 24.765 15.24) (width 0.4) (layer F.Cu) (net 23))
 (segment (start 24.765 15.24) (end 19.812 15.24) (width 0.4) (layer F.Cu) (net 23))
 (segment (start 23.495 27.56) (end 25.145 27.56) (width 0.4) (layer F.Cu) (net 23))
 (segment (start 23.876 13.97) (end 22.606 13.97) (width 0.4) (layer F.Cu) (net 25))
 (segment (start 22.606 13.97) (end 22.606 13.142) (width 0.4) (layer F.Cu) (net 25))
 (segment (start 30.48 19.05) (end 25.4 13.97) (width 0.4) (layer F.Cu) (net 25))
 (segment (start 25.4 13.97) (end 23.876 13.97) (width 0.4) (layer F.Cu) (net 25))
 (segment (start 23.495 29.56) (end 25.05 29.56) (width 0.4) (layer F.Cu) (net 25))
 (segment (start 25.05 29.56) (end 30.48 24.13) (width 0.4) (layer F.Cu) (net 25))
 (segment (start 30.48 24.13) (end 30.48 19.05) (width 0.4) (layer F.Cu) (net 25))
 (segment (start 6.985 26.035) (end 5.715 24.765) (width 0.4) (layer F.Cu) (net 16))
 (segment (start 9.495 27.56) (end 7.875 27.56) (width 0.4) (layer F.Cu) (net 16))
 (segment (start 7.875 27.56) (end 6.985 26.67) (width 0.4) (layer F.Cu) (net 16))
 (segment (start 6.985 26.67) (end 6.985 26.035) (width 0.4) (layer F.Cu) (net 16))
 (segment (start 7.62 27.305) (end 9.24 27.305) (width 0.4) (layer F.Cu) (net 16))
 (segment (start 9.24 27.305) (end 9.495 27.56) (width 0.4) (layer F.Cu) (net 16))
 (segment (start 12.065 5.98678) (end 12.065 5.08) (width 0.4) (layer F.Cu) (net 5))
 (segment (start 14.605 3.937) (end 14.605 2.54) (width 0.4) (layer F.Cu) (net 5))
 (segment (start 14.097 4.445) (end 14.605 3.937) (width 0.4) (layer F.Cu) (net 5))
 (segment (start 12.7 4.445) (end 14.097 4.445) (width 0.4) (layer F.Cu) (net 5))
 (segment (start 12.065 5.08) (end 12.7 4.445) (width 0.4) (layer F.Cu) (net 5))
 (segment (start 15.875 5.98678) (end 15.875 5.08) (width 0.4) (layer F.Cu) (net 3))
 (segment (start 17.145 4.191) (end 17.145 2.54) (width 0.4) (layer F.Cu) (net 3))
 (segment (start 16.891 4.445) (end 17.145 4.191) (width 0.4) (layer F.Cu) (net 3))
 (segment (start 16.51 4.445) (end 16.891 4.445) (width 0.4) (layer F.Cu) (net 3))
 (segment (start 15.875 5.08) (end 16.51 4.445) (width 0.4) (layer F.Cu) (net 3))
 (segment (start 19.685 5.98678) (end 19.685 2.54) (width 0.4) (layer F.Cu) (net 10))
 (segment (start 22.86 4.445) (end 22.479 4.445) (width 0.4) (layer F.Cu) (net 11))
 (segment (start 22.225 4.191) (end 22.225 2.54) (width 0.4) (layer F.Cu) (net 11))
 (segment (start 22.479 4.445) (end 22.225 4.191) (width 0.4) (layer F.Cu) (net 11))
 (segment (start 23.495 5.98678) (end 23.495 5.08) (width 0.4) (layer F.Cu) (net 11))
 (segment (start 23.495 5.08) (end 22.86 4.445) (width 0.4) (layer F.Cu) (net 11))
 (segment (start 27.94 34.605) (end 27.94 35.56) (width 0.4) (layer F.Cu) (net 18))
 (segment (start 23.495 35.56) (end 27.94 35.56) (width 0.4) (layer F.Cu) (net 18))
 (segment (start 27.94 35.56) (end 32.17418 35.56) (width 0.4) (layer F.Cu) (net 18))
 (segment (start 32.17418 35.56) (end 32.385 35.34918) (width 0.4) (layer F.Cu) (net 18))
 (segment (start 23.70582 35.34918) (end 23.495 35.56) (width 0.4) (layer F.Cu) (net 18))
 (segment (start 4.255 31.56) (end 9.495 31.56) (width 0.4) (layer F.Cu) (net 27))
 (segment (start 1.905 29.21) (end 4.255 31.56) (width 0.4) (layer F.Cu) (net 27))
 (segment (start 1.905 29.21) (end 1.27 28.575) (width 0.4) (layer F.Cu) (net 27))
 (segment (start 1.27 15.875) (end 1.905 15.24) (width 0.4) (layer F.Cu) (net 27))
 (segment (start 1.27 28.575) (end 1.27 15.875) (width 0.4) (layer F.Cu) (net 27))
 (segment (start 1.905 13.015) (end 1.905 15.24) (width 0.4) (layer F.Cu) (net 27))
 (segment (start 36.068 15.494) (end 36.068 4.826) (width 0.4) (layer F.Cu) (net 17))
 (segment (start 35.24 16.322) (end 36.068 15.494) (width 0.4) (layer F.Cu) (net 17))
 (segment (start 36.068 3.81) (end 34.798 2.54) (width 0.4) (layer F.Cu) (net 17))
 (segment (start 36.068 4.826) (end 36.068 3.81) (width 0.4) (layer F.Cu) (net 17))
 (segment (start 21.59 36.83) (end 21.844 37.084) (width 0.4) (layer F.Cu) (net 17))
 (segment (start 33.528 37.084) (end 33.782 36.83) (width 0.4) (layer F.Cu) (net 17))
 (segment (start 21.844 37.084) (end 33.528 37.084) (width 0.4) (layer F.Cu) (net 17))
 (segment (start 35.24 21.082) (end 35.24 16.322) (width 0.4) (layer F.Cu) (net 17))
 (segment (start 35.24 21.082) (end 35.24 35.372) (width 0.4) (layer F.Cu) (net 17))
 (segment (start 35.24 35.372) (end 33.782 36.83) (width 0.4) (layer F.Cu) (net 17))
 (segment (start 21.59 36.83) (end 10.32 25.56) (width 0.4) (layer F.Cu) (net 17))
 (segment (start 10.32 25.56) (end 9.495 25.56) (width 0.4) (layer F.Cu) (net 17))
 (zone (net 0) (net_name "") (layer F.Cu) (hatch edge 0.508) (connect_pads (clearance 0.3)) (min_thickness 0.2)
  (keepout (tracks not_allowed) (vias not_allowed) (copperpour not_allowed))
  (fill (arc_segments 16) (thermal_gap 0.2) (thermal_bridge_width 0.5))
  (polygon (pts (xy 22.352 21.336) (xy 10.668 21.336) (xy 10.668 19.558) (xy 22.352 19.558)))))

